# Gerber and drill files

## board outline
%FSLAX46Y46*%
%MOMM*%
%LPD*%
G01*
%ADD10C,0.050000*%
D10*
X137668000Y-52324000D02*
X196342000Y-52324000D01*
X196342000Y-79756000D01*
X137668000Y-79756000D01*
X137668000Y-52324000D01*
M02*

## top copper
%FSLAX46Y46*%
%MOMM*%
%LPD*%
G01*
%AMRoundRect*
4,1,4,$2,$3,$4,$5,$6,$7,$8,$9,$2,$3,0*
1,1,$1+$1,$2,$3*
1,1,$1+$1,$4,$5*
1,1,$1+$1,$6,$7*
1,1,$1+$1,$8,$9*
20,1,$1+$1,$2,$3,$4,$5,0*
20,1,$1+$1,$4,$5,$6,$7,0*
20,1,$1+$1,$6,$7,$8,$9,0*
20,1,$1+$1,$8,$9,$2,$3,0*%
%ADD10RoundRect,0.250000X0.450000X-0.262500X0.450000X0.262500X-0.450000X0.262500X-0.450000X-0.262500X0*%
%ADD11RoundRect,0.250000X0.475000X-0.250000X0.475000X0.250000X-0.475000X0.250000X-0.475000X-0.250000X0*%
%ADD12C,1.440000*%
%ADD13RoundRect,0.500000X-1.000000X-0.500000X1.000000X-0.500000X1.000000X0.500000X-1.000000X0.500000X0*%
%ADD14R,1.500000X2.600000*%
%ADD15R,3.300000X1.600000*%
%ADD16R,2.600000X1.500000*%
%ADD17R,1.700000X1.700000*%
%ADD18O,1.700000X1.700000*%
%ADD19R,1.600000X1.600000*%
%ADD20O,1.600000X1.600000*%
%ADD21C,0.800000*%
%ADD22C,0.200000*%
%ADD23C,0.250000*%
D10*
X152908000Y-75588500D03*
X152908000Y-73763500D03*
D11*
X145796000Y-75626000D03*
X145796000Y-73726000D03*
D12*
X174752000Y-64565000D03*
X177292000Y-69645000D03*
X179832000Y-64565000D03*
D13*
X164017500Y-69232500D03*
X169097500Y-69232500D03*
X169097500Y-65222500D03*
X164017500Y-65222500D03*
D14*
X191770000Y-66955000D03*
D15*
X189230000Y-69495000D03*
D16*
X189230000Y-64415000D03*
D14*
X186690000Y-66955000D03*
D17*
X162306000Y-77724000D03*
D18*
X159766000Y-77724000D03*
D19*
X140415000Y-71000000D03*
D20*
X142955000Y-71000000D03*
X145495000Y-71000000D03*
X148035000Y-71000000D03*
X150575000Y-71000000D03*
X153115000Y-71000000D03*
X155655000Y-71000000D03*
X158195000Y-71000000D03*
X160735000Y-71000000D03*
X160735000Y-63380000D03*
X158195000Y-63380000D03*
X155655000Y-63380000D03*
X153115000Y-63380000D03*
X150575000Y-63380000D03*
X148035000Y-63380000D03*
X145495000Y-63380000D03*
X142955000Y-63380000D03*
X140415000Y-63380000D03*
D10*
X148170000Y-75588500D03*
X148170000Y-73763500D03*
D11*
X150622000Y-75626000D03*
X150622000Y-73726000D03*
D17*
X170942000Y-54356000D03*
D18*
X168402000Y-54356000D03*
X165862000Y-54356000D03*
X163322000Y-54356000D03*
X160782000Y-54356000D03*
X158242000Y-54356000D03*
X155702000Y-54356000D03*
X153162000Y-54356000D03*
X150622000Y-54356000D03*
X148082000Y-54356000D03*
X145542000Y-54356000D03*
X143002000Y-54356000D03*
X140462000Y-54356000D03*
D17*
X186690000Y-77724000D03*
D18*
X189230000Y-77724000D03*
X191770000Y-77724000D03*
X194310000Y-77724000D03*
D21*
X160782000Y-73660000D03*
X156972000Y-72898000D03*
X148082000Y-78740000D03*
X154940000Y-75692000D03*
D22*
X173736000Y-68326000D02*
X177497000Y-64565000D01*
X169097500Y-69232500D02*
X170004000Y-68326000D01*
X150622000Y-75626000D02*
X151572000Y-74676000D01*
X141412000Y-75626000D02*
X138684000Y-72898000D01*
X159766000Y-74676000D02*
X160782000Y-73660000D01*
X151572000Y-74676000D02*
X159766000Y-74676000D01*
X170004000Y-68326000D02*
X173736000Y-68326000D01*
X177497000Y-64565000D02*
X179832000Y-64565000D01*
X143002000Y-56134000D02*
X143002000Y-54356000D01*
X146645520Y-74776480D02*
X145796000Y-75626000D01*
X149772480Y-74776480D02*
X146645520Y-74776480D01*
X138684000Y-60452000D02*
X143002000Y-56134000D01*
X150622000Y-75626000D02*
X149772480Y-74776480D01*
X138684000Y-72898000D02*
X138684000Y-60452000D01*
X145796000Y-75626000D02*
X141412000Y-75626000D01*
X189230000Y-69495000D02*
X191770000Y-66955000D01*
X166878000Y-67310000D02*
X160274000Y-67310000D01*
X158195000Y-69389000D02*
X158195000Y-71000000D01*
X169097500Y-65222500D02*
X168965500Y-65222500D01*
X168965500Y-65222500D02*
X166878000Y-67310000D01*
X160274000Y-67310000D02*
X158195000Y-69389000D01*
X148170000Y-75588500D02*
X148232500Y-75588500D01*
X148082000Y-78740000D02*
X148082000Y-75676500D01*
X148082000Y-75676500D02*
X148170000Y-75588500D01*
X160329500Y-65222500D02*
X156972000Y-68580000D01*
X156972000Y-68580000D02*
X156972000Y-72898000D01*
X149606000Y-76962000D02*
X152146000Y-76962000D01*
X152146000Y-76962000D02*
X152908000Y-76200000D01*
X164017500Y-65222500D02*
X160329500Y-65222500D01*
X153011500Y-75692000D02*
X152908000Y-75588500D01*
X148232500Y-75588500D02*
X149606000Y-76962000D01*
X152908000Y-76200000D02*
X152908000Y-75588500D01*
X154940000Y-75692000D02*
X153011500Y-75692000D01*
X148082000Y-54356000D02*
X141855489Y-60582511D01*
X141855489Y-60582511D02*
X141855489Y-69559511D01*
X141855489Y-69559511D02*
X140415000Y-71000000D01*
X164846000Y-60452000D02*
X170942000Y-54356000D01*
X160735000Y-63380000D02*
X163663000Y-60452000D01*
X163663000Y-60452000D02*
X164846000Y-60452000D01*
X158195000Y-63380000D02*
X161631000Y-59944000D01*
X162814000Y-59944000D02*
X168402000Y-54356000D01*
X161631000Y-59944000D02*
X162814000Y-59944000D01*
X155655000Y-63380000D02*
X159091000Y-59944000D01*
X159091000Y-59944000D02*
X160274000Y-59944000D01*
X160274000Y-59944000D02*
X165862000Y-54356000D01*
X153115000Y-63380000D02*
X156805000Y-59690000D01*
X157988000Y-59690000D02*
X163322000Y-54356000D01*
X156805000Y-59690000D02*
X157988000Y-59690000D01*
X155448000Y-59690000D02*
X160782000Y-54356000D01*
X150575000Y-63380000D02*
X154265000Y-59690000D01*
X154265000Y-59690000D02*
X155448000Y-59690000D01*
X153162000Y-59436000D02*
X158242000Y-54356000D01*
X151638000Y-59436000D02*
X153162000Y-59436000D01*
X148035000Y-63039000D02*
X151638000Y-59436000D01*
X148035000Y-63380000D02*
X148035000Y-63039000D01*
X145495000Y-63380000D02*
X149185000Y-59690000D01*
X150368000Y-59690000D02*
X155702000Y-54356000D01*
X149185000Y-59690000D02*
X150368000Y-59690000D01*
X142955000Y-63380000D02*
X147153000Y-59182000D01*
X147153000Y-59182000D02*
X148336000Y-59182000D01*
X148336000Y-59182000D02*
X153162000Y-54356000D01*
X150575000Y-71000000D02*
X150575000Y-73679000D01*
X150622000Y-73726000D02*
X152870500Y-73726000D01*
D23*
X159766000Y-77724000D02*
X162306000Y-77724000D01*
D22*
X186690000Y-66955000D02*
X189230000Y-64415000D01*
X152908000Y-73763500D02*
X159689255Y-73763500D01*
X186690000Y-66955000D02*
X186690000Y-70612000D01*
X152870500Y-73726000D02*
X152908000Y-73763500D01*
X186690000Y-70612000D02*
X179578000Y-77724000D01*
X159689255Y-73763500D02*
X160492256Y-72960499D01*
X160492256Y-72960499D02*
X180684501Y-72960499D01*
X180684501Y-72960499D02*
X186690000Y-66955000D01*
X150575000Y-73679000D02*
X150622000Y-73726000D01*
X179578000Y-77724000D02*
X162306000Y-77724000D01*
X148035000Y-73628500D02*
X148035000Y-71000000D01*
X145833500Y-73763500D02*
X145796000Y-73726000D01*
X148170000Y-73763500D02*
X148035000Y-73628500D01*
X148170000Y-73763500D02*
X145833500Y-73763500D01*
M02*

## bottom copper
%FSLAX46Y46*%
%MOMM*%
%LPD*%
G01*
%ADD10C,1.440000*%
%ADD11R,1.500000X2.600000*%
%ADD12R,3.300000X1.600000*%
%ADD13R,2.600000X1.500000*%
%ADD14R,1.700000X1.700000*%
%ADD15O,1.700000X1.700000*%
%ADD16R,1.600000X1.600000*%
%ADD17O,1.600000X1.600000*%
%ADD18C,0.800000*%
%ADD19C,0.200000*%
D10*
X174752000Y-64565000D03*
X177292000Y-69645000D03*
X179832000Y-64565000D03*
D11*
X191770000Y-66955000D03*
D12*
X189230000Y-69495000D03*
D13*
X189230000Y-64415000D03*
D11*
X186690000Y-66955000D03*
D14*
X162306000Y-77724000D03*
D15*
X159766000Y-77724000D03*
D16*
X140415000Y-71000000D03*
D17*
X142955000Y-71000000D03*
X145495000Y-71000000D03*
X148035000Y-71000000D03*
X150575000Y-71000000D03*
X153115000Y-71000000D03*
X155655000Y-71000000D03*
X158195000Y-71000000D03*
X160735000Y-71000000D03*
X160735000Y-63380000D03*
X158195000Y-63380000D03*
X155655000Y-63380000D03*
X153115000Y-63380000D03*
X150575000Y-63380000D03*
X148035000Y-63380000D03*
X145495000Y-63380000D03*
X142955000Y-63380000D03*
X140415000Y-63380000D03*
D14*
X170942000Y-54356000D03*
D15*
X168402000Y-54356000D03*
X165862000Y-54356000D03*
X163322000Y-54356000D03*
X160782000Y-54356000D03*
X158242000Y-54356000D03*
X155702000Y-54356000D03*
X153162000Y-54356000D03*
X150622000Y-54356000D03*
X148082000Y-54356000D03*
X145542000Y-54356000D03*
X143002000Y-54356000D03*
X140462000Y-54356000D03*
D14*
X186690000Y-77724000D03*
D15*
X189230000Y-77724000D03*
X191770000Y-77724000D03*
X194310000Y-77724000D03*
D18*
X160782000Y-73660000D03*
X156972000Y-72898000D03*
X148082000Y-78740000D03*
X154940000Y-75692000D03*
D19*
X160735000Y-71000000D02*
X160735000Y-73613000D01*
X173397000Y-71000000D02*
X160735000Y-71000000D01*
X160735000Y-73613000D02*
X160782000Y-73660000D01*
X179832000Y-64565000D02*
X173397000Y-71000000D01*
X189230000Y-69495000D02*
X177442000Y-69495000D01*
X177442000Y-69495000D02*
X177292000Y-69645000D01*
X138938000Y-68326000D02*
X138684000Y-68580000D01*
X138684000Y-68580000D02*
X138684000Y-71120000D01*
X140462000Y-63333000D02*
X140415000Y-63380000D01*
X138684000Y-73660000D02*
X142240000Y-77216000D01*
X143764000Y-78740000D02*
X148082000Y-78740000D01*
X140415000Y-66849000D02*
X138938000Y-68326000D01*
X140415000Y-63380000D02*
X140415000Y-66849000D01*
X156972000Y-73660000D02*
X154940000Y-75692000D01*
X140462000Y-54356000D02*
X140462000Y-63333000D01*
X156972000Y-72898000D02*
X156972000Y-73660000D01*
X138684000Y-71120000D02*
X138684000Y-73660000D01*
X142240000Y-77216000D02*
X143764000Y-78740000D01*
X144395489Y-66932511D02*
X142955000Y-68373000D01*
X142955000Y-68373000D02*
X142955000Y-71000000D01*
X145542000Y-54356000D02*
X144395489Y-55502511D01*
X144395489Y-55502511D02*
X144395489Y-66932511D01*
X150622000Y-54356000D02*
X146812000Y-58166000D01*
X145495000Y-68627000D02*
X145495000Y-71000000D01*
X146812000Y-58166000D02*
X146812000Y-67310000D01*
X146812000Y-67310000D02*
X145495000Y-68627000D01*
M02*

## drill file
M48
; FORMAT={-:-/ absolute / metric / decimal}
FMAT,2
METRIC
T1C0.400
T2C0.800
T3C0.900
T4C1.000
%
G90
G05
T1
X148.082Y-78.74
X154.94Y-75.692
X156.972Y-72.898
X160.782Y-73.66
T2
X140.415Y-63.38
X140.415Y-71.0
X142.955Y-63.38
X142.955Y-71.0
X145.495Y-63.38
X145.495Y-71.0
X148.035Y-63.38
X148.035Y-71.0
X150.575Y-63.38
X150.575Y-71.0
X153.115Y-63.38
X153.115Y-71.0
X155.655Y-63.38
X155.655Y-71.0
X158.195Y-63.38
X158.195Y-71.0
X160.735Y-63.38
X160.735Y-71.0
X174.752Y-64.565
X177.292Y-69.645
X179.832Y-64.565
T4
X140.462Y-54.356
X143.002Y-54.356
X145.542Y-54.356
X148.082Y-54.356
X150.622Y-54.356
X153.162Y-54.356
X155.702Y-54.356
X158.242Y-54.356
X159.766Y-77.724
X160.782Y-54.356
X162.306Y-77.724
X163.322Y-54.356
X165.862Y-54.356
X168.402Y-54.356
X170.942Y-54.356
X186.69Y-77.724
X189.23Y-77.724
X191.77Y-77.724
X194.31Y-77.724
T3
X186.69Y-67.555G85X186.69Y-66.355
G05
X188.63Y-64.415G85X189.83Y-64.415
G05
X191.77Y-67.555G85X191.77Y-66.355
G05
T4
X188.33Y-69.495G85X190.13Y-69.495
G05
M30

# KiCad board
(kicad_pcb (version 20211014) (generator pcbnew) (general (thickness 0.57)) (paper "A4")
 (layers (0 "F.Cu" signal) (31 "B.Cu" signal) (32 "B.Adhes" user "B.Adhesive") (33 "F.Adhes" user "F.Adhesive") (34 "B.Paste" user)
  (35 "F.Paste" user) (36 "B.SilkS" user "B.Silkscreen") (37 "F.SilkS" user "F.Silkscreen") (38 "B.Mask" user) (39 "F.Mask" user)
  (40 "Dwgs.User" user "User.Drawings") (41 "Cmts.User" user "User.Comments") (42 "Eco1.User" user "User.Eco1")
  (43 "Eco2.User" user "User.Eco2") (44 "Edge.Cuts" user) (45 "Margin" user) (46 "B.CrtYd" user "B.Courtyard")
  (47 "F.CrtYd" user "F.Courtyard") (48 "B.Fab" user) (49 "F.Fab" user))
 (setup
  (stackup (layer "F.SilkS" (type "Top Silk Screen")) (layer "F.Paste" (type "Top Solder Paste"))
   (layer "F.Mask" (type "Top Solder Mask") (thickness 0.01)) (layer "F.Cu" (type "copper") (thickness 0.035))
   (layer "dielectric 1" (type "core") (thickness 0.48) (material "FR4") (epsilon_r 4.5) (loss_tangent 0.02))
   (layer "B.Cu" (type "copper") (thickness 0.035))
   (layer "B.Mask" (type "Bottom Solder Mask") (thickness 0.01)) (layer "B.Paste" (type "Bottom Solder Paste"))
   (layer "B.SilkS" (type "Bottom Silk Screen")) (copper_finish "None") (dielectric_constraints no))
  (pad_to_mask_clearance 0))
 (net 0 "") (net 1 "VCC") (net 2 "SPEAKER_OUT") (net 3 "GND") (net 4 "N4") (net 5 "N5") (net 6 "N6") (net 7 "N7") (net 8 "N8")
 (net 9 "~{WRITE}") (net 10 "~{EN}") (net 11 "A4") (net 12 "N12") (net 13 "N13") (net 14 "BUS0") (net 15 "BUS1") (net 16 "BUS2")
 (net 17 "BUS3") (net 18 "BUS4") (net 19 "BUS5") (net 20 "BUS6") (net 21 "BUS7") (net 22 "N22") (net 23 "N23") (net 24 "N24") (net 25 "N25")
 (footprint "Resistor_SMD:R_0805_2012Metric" (layer "F.Cu") (at 152.908 74.676 90)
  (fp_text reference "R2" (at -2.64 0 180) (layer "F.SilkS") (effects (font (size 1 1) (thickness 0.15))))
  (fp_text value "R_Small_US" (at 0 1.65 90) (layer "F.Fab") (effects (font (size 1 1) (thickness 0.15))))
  (pad "1" smd roundrect locked (at -0.9125 0 90) (size 1.025 1.4) (layers "F.Cu" "F.Paste" "F.Mask") (roundrect_rratio 0.243902)
   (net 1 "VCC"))
  (pad "2" smd roundrect locked (at 0.9125 0 90) (size 1.025 1.4) (layers "F.Cu" "F.Paste" "F.Mask") (roundrect_rratio 0.243902)
   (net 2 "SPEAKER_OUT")))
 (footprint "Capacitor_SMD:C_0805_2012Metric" (layer "F.Cu") (at 145.796 74.676 90)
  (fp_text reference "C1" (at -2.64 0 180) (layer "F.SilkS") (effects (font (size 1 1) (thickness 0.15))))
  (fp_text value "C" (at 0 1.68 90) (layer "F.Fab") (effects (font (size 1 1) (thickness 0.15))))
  (pad "1" smd roundrect locked (at -0.95 0 90) (size 1 1.45) (layers "F.Cu" "F.Paste" "F.Mask") (roundrect_rratio 0.25) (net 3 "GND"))
  (pad "2" smd roundrect locked (at 0.95 0 90) (size 1 1.45) (layers "F.Cu" "F.Paste" "F.Mask") (roundrect_rratio 0.25) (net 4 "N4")))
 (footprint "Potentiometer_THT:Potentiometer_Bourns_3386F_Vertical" (layer "F.Cu") (at 174.752 64.565 -90)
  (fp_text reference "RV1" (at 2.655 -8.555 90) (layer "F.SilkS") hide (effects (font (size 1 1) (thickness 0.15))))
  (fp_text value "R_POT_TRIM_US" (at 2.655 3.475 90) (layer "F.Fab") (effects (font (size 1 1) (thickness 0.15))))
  (pad "1" thru_hole circle (at 0 0 270) (size 1.44 1.44) (drill 0.8) (layers *.Cu *.Mask) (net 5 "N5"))
  (pad "2" thru_hole circle (at 5.08 -2.54 270) (size 1.44 1.44) (drill 0.8) (layers *.Cu *.Mask) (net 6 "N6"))
  (pad "3" thru_hole circle (at 0 -5.08 270) (size 1.44 1.44) (drill 0.8) (layers *.Cu *.Mask) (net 3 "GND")))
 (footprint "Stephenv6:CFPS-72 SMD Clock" (layer "F.Cu") (at 166.6075 57.0525)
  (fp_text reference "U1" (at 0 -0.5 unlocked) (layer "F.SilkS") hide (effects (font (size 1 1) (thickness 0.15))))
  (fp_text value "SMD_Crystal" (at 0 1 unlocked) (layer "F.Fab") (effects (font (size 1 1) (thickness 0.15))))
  (pad "1" smd roundrect (at -2.59 12.18) (size 3 2) (layers "F.Cu" "F.Paste" "F.Mask") (roundrect_rratio 0.25) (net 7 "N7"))
  (pad "2" smd roundrect (at 2.49 12.18) (size 3 2) (layers "F.Cu" "F.Paste" "F.Mask") (roundrect_rratio 0.25) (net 3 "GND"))
  (pad "3" smd roundrect (at 2.49 8.17) (size 3 2) (layers "F.Cu" "F.Paste" "F.Mask") (roundrect_rratio 0.25) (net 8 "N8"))
  (pad "4" smd roundrect (at -2.59 8.17) (size 3 2) (layers "F.Cu" "F.Paste" "F.Mask") (roundrect_rratio 0.25) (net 1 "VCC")))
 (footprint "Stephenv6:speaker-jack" (layer "F.Cu") (at 189.2 57.655467)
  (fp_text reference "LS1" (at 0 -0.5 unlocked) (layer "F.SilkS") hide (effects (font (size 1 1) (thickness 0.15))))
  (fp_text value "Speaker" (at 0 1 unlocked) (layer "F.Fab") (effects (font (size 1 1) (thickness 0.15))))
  (pad "R1" thru_hole rect (at 2.57 9.299533 180) (size 1.5 2.6) (drill oval 0.9 2.1) (layers *.Cu *.Mask) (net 6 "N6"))
  (pad "R2" thru_hole rect (at 0.03 11.839533 90) (size 1.6 3.3) (drill oval 1 2.8) (layers *.Cu *.Mask) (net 6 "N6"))
  (pad "S" thru_hole rect (at 0.03 6.759533 90) (size 1.5 2.6) (drill oval 0.9 2.1) (layers *.Cu *.Mask) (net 2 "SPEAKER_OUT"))
  (pad "T" thru_hole rect (at -2.51 9.299533 180) (size 1.5 2.6) (drill oval 0.9 2.1) (layers *.Cu *.Mask) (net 2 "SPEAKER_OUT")))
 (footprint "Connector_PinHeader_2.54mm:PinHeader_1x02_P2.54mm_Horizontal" (layer "F.Cu") (at 162.306 77.724 -90)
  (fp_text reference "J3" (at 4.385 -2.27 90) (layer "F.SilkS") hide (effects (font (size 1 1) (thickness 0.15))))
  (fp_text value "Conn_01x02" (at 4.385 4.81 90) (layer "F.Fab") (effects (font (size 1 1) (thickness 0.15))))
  (pad "1" thru_hole rect locked (at 0 0 270) (size 1.7 1.7) (drill 1) (layers *.Cu *.Mask) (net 2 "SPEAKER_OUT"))
  (pad "2" thru_hole oval locked (at 0 2.54 270) (size 1.7 1.7) (drill 1) (layers *.Cu *.Mask) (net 2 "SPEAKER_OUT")))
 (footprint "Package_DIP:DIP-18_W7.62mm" (layer "F.Cu") (at 140.415 71 90)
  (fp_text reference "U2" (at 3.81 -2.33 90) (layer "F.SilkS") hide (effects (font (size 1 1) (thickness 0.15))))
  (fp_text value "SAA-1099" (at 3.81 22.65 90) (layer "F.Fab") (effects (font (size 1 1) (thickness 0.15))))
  (pad "1" thru_hole rect locked (at 0 0 90) (size 1.6 1.6) (drill 0.8) (layers *.Cu *.Mask) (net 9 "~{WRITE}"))
  (pad "2" thru_hole oval locked (at 0 2.54 90) (size 1.6 1.6) (drill 0.8) (layers *.Cu *.Mask) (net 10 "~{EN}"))
  (pad "3" thru_hole oval locked (at 0 5.08 90) (size 1.6 1.6) (drill 0.8) (layers *.Cu *.Mask) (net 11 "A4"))
  (pad "4" thru_hole oval locked (at 0 7.62 90) (size 1.6 1.6) (drill 0.8) (layers *.Cu *.Mask) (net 4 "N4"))
  (pad "5" thru_hole oval locked (at 0 10.16 90) (size 1.6 1.6) (drill 0.8) (layers *.Cu *.Mask) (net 2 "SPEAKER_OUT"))
  (pad "6" thru_hole oval locked (at 0 12.7 90) (size 1.6 1.6) (drill 0.8) (layers *.Cu *.Mask) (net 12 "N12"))
  (pad "7" thru_hole oval locked (at 0 15.24 90) (size 1.6 1.6) (drill 0.8) (layers *.Cu *.Mask) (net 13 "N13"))
  (pad "8" thru_hole oval locked (at 0 17.78 90) (size 1.6 1.6) (drill 0.8) (layers *.Cu *.Mask) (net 8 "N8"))
  (pad "9" thru_hole oval locked (at 0 20.32 90) (size 1.6 1.6) (drill 0.8) (layers *.Cu *.Mask) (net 3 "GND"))
  (pad "10" thru_hole oval locked (at 7.62 20.32 90) (size 1.6 1.6) (drill 0.8) (layers *.Cu *.Mask) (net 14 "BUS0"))
  (pad "11" thru_hole oval locked (at 7.62 17.78 90) (size 1.6 1.6) (drill 0.8) (layers *.Cu *.Mask) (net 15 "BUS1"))
  (pad "12" thru_hole oval locked (at 7.62 15.24 90) (size 1.6 1.6) (drill 0.8) (layers *.Cu *.Mask) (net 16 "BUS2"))
  (pad "13" thru_hole oval locked (at 7.62 12.7 90) (size 1.6 1.6) (drill 0.8) (layers *.Cu *.Mask) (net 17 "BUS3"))
  (pad "14" thru_hole oval locked (at 7.62 10.16 90) (size 1.6 1.6) (drill 0.8) (layers *.Cu *.Mask) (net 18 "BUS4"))
  (pad "15" thru_hole oval locked (at 7.62 7.62 90) (size 1.6 1.6) (drill 0.8) (layers *.Cu *.Mask) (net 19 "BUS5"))
  (pad "16" thru_hole oval locked (at 7.62 5.08 90) (size 1.6 1.6) (drill 0.8) (layers *.Cu *.Mask) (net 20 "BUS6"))
  (pad "17" thru_hole oval locked (at 7.62 2.54 90) (size 1.6 1.6) (drill 0.8) (layers *.Cu *.Mask) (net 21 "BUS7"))
  (pad "18" thru_hole oval locked (at 7.62 0 90) (size 1.6 1.6) (drill 0.8) (layers *.Cu *.Mask) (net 1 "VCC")))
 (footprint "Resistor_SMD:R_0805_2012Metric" (layer "F.Cu") (at 148.17 74.676 90)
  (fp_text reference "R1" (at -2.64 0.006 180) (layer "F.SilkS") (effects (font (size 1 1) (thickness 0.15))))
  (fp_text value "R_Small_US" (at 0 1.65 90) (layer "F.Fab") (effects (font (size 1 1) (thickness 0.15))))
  (pad "1" smd roundrect locked (at -0.9125 0 90) (size 1.025 1.4) (layers "F.Cu" "F.Paste" "F.Mask") (roundrect_rratio 0.243902)
   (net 1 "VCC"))
  (pad "2" smd roundrect locked (at 0.9125 0 90) (size 1.025 1.4) (layers "F.Cu" "F.Paste" "F.Mask") (roundrect_rratio 0.243902)
   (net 4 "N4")))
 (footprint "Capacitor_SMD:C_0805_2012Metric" (layer "F.Cu") (at 150.622 74.676 90)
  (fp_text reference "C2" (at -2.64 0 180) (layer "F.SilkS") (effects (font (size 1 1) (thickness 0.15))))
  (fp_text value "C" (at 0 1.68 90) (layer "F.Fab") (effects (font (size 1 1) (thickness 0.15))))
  (pad "1" smd roundrect locked (at -0.95 0 90) (size 1 1.45) (layers "F.Cu" "F.Paste" "F.Mask") (roundrect_rratio 0.25) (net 3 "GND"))
  (pad "2" smd roundrect locked (at 0.95 0 90) (size 1 1.45) (layers "F.Cu" "F.Paste" "F.Mask") (roundrect_rratio 0.25)
   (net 2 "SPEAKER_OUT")))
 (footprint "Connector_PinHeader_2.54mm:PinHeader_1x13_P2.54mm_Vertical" (layer "B.Cu") (at 170.942 54.356 90)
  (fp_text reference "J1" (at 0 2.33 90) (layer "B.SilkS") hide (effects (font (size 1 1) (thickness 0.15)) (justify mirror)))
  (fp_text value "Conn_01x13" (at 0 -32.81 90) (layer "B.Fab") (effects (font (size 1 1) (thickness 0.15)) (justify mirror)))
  (pad "1" thru_hole rect locked (at 0 0 90) (size 1.7 1.7) (drill 1) (layers *.Cu *.Mask) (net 14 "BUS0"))
  (pad "2" thru_hole oval locked (at 0 -2.54 90) (size 1.7 1.7) (drill 1) (layers *.Cu *.Mask) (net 15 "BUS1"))
  (pad "3" thru_hole oval locked (at 0 -5.08 90) (size 1.7 1.7) (drill 1) (layers *.Cu *.Mask) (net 16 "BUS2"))
  (pad "4" thru_hole oval locked (at 0 -7.62 90) (size 1.7 1.7) (drill 1) (layers *.Cu *.Mask) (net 17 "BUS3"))
  (pad "5" thru_hole oval locked (at 0 -10.16 90) (size 1.7 1.7) (drill 1) (layers *.Cu *.Mask) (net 18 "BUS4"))
  (pad "6" thru_hole oval locked (at 0 -12.7 90) (size 1.7 1.7) (drill 1) (layers *.Cu *.Mask) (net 19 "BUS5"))
  (pad "7" thru_hole oval locked (at 0 -15.24 90) (size 1.7 1.7) (drill 1) (layers *.Cu *.Mask) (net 20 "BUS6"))
  (pad "8" thru_hole oval locked (at 0 -17.78 90) (size 1.7 1.7) (drill 1) (layers *.Cu *.Mask) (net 21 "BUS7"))
  (pad "9" thru_hole oval locked (at 0 -20.32 90) (size 1.7 1.7) (drill 1) (layers *.Cu *.Mask) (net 11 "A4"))
  (pad "10" thru_hole oval locked (at 0 -22.86 90) (size 1.7 1.7) (drill 1) (layers *.Cu *.Mask) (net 9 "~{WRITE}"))
  (pad "11" thru_hole oval locked (at 0 -25.4 90) (size 1.7 1.7) (drill 1) (layers *.Cu *.Mask) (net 10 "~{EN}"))
  (pad "12" thru_hole oval locked (at 0 -27.94 90) (size 1.7 1.7) (drill 1) (layers *.Cu *.Mask) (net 3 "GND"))
  (pad "13" thru_hole oval locked (at 0 -30.48 90) (size 1.7 1.7) (drill 1) (layers *.Cu *.Mask) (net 1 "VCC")))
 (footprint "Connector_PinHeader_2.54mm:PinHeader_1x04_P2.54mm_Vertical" (layer "B.Cu") (at 186.69 77.724 -90)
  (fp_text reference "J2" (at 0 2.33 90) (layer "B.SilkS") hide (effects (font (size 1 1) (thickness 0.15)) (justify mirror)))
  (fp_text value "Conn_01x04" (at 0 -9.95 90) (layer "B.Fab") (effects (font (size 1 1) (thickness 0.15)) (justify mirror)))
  (pad "1" thru_hole rect locked (at 0 0 270) (size 1.7 1.7) (drill 1) (layers *.Cu *.Mask) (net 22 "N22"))
  (pad "2" thru_hole oval locked (at 0 -2.54 270) (size 1.7 1.7) (drill 1) (layers *.Cu *.Mask) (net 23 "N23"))
  (pad "3" thru_hole oval locked (at 0 -5.08 270) (size 1.7 1.7) (drill 1) (layers *.Cu *.Mask) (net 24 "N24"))
  (pad "4" thru_hole oval locked (at 0 -7.62 270) (size 1.7 1.7) (drill 1) (layers *.Cu *.Mask) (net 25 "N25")))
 (gr_rect (start 137.668 52.324) (end 196.342 79.756) (layer "Edge.Cuts") (width 0.05) (fill none))
 (segment (start 173.736 68.326) (end 177.497 64.565) (width 0.2) (layer "F.Cu") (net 3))
 (segment (start 169.0975 69.2325) (end 170.004 68.326) (width 0.2) (layer "F.Cu") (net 3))
 (segment (start 150.622 75.626) (end 151.572 74.676) (width 0.2) (layer "F.Cu") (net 3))
 (segment (start 141.412 75.626) (end 138.684 72.898) (width 0.2) (layer "F.Cu") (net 3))
 (segment (start 159.766 74.676) (end 160.782 73.66) (width 0.2) (layer "F.Cu") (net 3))
 (segment (start 151.572 74.676) (end 159.766 74.676) (width 0.2) (layer "F.Cu") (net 3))
 (segment (start 170.004 68.326) (end 173.736 68.326) (width 0.2) (layer "F.Cu") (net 3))
 (segment (start 177.497 64.565) (end 179.832 64.565) (width 0.2) (layer "F.Cu") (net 3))
 (segment (start 143.002 56.134) (end 143.002 54.356) (width 0.2) (layer "F.Cu") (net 3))
 (segment (start 146.64552 74.77648) (end 145.796 75.626) (width 0.2) (layer "F.Cu") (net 3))
 (segment (start 149.77248 74.77648) (end 146.64552 74.77648) (width 0.2) (layer "F.Cu") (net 3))
 (segment (start 138.684 60.452) (end 143.002 56.134) (width 0.2) (layer "F.Cu") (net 3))
 (segment (start 150.622 75.626) (end 149.77248 74.77648) (width 0.2) (layer "F.Cu") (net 3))
 (segment (start 138.684 72.898) (end 138.684 60.452) (width 0.2) (layer "F.Cu") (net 3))
 (segment (start 145.796 75.626) (end 141.412 75.626) (width 0.2) (layer "F.Cu") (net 3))
 (via (at 160.782 73.66) (size 0.8) (drill 0.4) (layers "F.Cu" "B.Cu") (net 3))
 (segment (start 160.735 71) (end 160.735 73.613) (width 0.2) (layer "B.Cu") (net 3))
 (segment (start 173.397 71) (end 160.735 71) (width 0.2) (layer "B.Cu") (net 3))
 (segment (start 160.735 73.613) (end 160.782 73.66) (width 0.2) (layer "B.Cu") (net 3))
 (segment (start 179.832 64.565) (end 173.397 71) (width 0.2) (layer "B.Cu") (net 3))
 (segment (start 189.23 69.495) (end 191.77 66.955) (width 0.2) (layer "F.Cu") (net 6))
 (segment (start 189.23 69.495) (end 177.442 69.495) (width 0.2) (layer "B.Cu") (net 6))
 (segment (start 177.442 69.495) (end 177.292 69.645) (width 0.2) (layer "B.Cu") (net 6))
 (segment (start 166.878 67.31) (end 160.274 67.31) (width 0.2) (layer "F.Cu") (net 8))
 (segment (start 158.195 69.389) (end 158.195 71) (width 0.2) (layer "F.Cu") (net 8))
 (segment (start 169.0975 65.2225) (end 168.9655 65.2225) (width 0.2) (layer "F.Cu") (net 8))
 (segment (start 168.9655 65.2225) (end 166.878 67.31) (width 0.2) (layer "F.Cu") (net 8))
 (segment (start 160.274 67.31) (end 158.195 69.389) (width 0.2) (layer "F.Cu") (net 8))
 (segment (start 148.17 75.5885) (end 148.2325 75.5885) (width 0.2) (layer "F.Cu") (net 1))
 (segment (start 148.082 78.74) (end 148.082 75.6765) (width 0.2) (layer "F.Cu") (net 1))
 (segment (start 148.082 75.6765) (end 148.17 75.5885) (width 0.2) (layer "F.Cu") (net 1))
 (segment (start 160.3295 65.2225) (end 156.972 68.58) (width 0.2) (layer "F.Cu") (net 1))
 (segment (start 156.972 68.58) (end 156.972 72.898) (width 0.2) (layer "F.Cu") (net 1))
 (segment (start 149.606 76.962) (end 152.146 76.962) (width 0.2) (layer "F.Cu") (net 1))
 (segment (start 152.146 76.962) (end 152.908 76.2) (width 0.2) (layer "F.Cu") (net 1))
 (segment (start 164.0175 65.2225) (end 160.3295 65.2225) (width 0.2) (layer "F.Cu") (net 1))
 (segment (start 153.0115 75.692) (end 152.908 75.5885) (width 0.2) (layer "F.Cu") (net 1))
 (segment (start 148.2325 75.5885) (end 149.606 76.962) (width 0.2) (layer "F.Cu") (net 1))
 (segment (start 152.908 76.2) (end 152.908 75.5885) (width 0.2) (layer "F.Cu") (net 1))
 (segment (start 154.94 75.692) (end 153.0115 75.692) (width 0.2) (layer "F.Cu") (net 1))
 (via (at 156.972 72.898) (size 0.8) (drill 0.4) (layers "F.Cu" "B.Cu") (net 1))
 (via (at 148.082 78.74) (size 0.8) (drill 0.4) (layers "F.Cu" "B.Cu") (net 1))
 (via (at 154.94 75.692) (size 0.8) (drill 0.4) (layers "F.Cu" "B.Cu") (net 1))
 (segment (start 138.938 68.326) (end 138.684 68.58) (width 0.2) (layer "B.Cu") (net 1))
 (segment (start 138.684 68.58) (end 138.684 71.12) (width 0.2) (layer "B.Cu") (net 1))
 (segment (start 140.462 63.333) (end 140.415 63.38) (width 0.2) (layer "B.Cu") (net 1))
 (segment (start 138.684 73.66) (end 142.24 77.216) (width 0.2) (layer "B.Cu") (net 1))
 (segment (start 143.764 78.74) (end 148.082 78.74) (width 0.2) (layer "B.Cu") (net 1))
 (segment (start 140.415 66.849) (end 138.938 68.326) (width 0.2) (layer "B.Cu") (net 1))
 (segment (start 140.415 63.38) (end 140.415 66.849) (width 0.2) (layer "B.Cu") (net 1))
 (segment (start 156.972 73.66) (end 154.94 75.692) (width 0.2) (layer "B.Cu") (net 1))
 (segment (start 140.462 54.356) (end 140.462 63.333) (width 0.2) (layer "B.Cu") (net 1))
 (segment (start 156.972 72.898) (end 156.972 73.66) (width 0.2) (layer "B.Cu") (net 1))
 (segment (start 138.684 71.12) (end 138.684 73.66) (width 0.2) (layer "B.Cu") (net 1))
 (segment (start 142.24 77.216) (end 143.764 78.74) (width 0.2) (layer "B.Cu") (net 1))
 (segment (start 148.082 54.356) (end 141.855489 60.582511) (width 0.2) (layer "F.Cu") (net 9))
 (segment (start 141.855489 60.582511) (end 141.855489 69.559511) (width 0.2) (layer "F.Cu") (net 9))
 (segment (start 141.855489 69.559511) (end 140.415 71) (width 0.2) (layer "F.Cu") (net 9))
 (segment (start 144.395489 66.932511) (end 142.955 68.373) (width 0.2) (layer "B.Cu") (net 10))
 (segment (start 142.955 68.373) (end 142.955 71) (width 0.2) (layer "B.Cu") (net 10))
 (segment (start 145.542 54.356) (end 144.395489 55.502511) (width 0.2) (layer "B.Cu") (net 10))
 (segment (start 144.395489 55.502511) (end 144.395489 66.932511) (width 0.2) (layer "B.Cu") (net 10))
 (segment (start 164.846 60.452) (end 170.942 54.356) (width 0.2) (layer "F.Cu") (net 14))
 (segment (start 160.735 63.38) (end 163.663 60.452) (width 0.2) (layer "F.Cu") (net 14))
 (segment (start 163.663 60.452) (end 164.846 60.452) (width 0.2) (layer "F.Cu") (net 14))
 (segment (start 150.622 54.356) (end 146.812 58.166) (width 0.2) (layer "B.Cu") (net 11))
 (segment (start 145.495 68.627) (end 145.495 71) (width 0.2) (layer "B.Cu") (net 11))
 (segment (start 146.812 58.166) (end 146.812 67.31) (width 0.2) (layer "B.Cu") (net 11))
 (segment (start 146.812 67.31) (end 145.495 68.627) (width 0.2) (layer "B.Cu") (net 11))
 (segment (start 158.195 63.38) (end 161.631 59.944) (width 0.2) (layer "F.Cu") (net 15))
 (segment (start 162.814 59.944) (end 168.402 54.356) (width 0.2) (layer "F.Cu") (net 15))
 (segment (start 161.631 59.944) (end 162.814 59.944) (width 0.2) (layer "F.Cu") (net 15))
 (segment (start 155.655 63.38) (end 159.091 59.944) (width 0.2) (layer "F.Cu") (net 16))
 (segment (start 159.091 59.944) (end 160.274 59.944) (width 0.2) (layer "F.Cu") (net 16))
 (segment (start 160.274 59.944) (end 165.862 54.356) (width 0.2) (layer "F.Cu") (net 16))
 (segment (start 153.115 63.38) (end 156.805 59.69) (width 0.2) (layer "F.Cu") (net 17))
 (segment (start 157.988 59.69) (end 163.322 54.356) (width 0.2) (layer "F.Cu") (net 17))
 (segment (start 156.805 59.69) (end 157.988 59.69) (width 0.2) (layer "F.Cu") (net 17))
 (segment (start 155.448 59.69) (end 160.782 54.356) (width 0.2) (layer "F.Cu") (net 18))
 (segment (start 150.575 63.38) (end 154.265 59.69) (width 0.2) (layer "F.Cu") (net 18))
 (segment (start 154.265 59.69) (end 155.448 59.69) (width 0.2) (layer "F.Cu") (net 18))
 (segment (start 153.162 59.436) (end 158.242 54.356) (width 0.2) (layer "F.Cu") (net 19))
 (segment (start 151.638 59.436) (end 153.162 59.436) (width 0.2) (layer "F.Cu") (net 19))
 (segment (start 148.035 63.039) (end 151.638 59.436) (width 0.2) (layer "F.Cu") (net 19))
 (segment (start 148.035 63.38) (end 148.035 63.039) (width 0.2) (layer "F.Cu") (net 19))
 (segment (start 145.495 63.38) (end 149.185 59.69) (width 0.2) (layer "F.Cu") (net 20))
 (segment (start 150.368 59.69) (end 155.702 54.356) (width 0.2) (layer "F.Cu") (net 20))
 (segment (start 149.185 59.69) (end 150.368 59.69) (width 0.2) (layer "F.Cu") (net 20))
 (segment (start 142.955 63.38) (end 147.153 59.182) (width 0.2) (layer "F.Cu") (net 21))
 (segment (start 147.153 59.182) (end 148.336 59.182) (width 0.2) (layer "F.Cu") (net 21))
 (segment (start 148.336 59.182) (end 153.162 54.356) (width 0.2) (layer "F.Cu") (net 21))
 (segment (start 150.575 71) (end 150.575 73.679) (width 0.2) (layer "F.Cu") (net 2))
 (segment (start 150.622 73.726) (end 152.8705 73.726) (width 0.2) (layer "F.Cu") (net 2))
 (segment (start 159.766 77.724) (end 162.306 77.724) (width 0.25) (layer "F.Cu") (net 2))
 (segment (start 186.69 66.955) (end 189.23 64.415) (width 0.2) (layer "F.Cu") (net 2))
 (segment (start 152.908 73.7635) (end 159.689255 73.7635) (width 0.2) (layer "F.Cu") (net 2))
 (segment (start 186.69 66.955) (end 186.69 70.612) (width 0.2) (layer "F.Cu") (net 2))
 (segment (start 152.8705 73.726) (end 152.908 73.7635) (width 0.2) (layer "F.Cu") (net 2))
 (segment (start 186.69 70.612) (end 179.578 77.724) (width 0.2) (layer "F.Cu") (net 2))
 (segment (start 159.689255 73.7635) (end 160.492256 72.960499) (width 0.2) (layer "F.Cu") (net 2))
 (segment (start 160.492256 72.960499) (end 180.684501 72.960499) (width 0.2) (layer "F.Cu") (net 2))
 (segment (start 180.684501 72.960499) (end 186.69 66.955) (width 0.2) (layer "F.Cu") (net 2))
 (segment (start 150.575 73.679) (end 150.622 73.726) (width 0.2) (layer "F.Cu") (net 2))
 (segment (start 179.578 77.724) (end 162.306 77.724) (width 0.2) (layer "F.Cu") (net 2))
 (segment (start 148.035 73.6285) (end 148.035 71) (width 0.2) (layer "F.Cu") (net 4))
 (segment (start 145.8335 73.7635) (end 145.796 73.726) (width 0.2) (layer "F.Cu") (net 4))
 (segment (start 148.17 73.7635) (end 148.035 73.6285) (width 0.2) (layer "F.Cu") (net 4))
 (segment (start 148.17 73.7635) (end 145.8335 73.7635) (width 0.2) (layer "F.Cu") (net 4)))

